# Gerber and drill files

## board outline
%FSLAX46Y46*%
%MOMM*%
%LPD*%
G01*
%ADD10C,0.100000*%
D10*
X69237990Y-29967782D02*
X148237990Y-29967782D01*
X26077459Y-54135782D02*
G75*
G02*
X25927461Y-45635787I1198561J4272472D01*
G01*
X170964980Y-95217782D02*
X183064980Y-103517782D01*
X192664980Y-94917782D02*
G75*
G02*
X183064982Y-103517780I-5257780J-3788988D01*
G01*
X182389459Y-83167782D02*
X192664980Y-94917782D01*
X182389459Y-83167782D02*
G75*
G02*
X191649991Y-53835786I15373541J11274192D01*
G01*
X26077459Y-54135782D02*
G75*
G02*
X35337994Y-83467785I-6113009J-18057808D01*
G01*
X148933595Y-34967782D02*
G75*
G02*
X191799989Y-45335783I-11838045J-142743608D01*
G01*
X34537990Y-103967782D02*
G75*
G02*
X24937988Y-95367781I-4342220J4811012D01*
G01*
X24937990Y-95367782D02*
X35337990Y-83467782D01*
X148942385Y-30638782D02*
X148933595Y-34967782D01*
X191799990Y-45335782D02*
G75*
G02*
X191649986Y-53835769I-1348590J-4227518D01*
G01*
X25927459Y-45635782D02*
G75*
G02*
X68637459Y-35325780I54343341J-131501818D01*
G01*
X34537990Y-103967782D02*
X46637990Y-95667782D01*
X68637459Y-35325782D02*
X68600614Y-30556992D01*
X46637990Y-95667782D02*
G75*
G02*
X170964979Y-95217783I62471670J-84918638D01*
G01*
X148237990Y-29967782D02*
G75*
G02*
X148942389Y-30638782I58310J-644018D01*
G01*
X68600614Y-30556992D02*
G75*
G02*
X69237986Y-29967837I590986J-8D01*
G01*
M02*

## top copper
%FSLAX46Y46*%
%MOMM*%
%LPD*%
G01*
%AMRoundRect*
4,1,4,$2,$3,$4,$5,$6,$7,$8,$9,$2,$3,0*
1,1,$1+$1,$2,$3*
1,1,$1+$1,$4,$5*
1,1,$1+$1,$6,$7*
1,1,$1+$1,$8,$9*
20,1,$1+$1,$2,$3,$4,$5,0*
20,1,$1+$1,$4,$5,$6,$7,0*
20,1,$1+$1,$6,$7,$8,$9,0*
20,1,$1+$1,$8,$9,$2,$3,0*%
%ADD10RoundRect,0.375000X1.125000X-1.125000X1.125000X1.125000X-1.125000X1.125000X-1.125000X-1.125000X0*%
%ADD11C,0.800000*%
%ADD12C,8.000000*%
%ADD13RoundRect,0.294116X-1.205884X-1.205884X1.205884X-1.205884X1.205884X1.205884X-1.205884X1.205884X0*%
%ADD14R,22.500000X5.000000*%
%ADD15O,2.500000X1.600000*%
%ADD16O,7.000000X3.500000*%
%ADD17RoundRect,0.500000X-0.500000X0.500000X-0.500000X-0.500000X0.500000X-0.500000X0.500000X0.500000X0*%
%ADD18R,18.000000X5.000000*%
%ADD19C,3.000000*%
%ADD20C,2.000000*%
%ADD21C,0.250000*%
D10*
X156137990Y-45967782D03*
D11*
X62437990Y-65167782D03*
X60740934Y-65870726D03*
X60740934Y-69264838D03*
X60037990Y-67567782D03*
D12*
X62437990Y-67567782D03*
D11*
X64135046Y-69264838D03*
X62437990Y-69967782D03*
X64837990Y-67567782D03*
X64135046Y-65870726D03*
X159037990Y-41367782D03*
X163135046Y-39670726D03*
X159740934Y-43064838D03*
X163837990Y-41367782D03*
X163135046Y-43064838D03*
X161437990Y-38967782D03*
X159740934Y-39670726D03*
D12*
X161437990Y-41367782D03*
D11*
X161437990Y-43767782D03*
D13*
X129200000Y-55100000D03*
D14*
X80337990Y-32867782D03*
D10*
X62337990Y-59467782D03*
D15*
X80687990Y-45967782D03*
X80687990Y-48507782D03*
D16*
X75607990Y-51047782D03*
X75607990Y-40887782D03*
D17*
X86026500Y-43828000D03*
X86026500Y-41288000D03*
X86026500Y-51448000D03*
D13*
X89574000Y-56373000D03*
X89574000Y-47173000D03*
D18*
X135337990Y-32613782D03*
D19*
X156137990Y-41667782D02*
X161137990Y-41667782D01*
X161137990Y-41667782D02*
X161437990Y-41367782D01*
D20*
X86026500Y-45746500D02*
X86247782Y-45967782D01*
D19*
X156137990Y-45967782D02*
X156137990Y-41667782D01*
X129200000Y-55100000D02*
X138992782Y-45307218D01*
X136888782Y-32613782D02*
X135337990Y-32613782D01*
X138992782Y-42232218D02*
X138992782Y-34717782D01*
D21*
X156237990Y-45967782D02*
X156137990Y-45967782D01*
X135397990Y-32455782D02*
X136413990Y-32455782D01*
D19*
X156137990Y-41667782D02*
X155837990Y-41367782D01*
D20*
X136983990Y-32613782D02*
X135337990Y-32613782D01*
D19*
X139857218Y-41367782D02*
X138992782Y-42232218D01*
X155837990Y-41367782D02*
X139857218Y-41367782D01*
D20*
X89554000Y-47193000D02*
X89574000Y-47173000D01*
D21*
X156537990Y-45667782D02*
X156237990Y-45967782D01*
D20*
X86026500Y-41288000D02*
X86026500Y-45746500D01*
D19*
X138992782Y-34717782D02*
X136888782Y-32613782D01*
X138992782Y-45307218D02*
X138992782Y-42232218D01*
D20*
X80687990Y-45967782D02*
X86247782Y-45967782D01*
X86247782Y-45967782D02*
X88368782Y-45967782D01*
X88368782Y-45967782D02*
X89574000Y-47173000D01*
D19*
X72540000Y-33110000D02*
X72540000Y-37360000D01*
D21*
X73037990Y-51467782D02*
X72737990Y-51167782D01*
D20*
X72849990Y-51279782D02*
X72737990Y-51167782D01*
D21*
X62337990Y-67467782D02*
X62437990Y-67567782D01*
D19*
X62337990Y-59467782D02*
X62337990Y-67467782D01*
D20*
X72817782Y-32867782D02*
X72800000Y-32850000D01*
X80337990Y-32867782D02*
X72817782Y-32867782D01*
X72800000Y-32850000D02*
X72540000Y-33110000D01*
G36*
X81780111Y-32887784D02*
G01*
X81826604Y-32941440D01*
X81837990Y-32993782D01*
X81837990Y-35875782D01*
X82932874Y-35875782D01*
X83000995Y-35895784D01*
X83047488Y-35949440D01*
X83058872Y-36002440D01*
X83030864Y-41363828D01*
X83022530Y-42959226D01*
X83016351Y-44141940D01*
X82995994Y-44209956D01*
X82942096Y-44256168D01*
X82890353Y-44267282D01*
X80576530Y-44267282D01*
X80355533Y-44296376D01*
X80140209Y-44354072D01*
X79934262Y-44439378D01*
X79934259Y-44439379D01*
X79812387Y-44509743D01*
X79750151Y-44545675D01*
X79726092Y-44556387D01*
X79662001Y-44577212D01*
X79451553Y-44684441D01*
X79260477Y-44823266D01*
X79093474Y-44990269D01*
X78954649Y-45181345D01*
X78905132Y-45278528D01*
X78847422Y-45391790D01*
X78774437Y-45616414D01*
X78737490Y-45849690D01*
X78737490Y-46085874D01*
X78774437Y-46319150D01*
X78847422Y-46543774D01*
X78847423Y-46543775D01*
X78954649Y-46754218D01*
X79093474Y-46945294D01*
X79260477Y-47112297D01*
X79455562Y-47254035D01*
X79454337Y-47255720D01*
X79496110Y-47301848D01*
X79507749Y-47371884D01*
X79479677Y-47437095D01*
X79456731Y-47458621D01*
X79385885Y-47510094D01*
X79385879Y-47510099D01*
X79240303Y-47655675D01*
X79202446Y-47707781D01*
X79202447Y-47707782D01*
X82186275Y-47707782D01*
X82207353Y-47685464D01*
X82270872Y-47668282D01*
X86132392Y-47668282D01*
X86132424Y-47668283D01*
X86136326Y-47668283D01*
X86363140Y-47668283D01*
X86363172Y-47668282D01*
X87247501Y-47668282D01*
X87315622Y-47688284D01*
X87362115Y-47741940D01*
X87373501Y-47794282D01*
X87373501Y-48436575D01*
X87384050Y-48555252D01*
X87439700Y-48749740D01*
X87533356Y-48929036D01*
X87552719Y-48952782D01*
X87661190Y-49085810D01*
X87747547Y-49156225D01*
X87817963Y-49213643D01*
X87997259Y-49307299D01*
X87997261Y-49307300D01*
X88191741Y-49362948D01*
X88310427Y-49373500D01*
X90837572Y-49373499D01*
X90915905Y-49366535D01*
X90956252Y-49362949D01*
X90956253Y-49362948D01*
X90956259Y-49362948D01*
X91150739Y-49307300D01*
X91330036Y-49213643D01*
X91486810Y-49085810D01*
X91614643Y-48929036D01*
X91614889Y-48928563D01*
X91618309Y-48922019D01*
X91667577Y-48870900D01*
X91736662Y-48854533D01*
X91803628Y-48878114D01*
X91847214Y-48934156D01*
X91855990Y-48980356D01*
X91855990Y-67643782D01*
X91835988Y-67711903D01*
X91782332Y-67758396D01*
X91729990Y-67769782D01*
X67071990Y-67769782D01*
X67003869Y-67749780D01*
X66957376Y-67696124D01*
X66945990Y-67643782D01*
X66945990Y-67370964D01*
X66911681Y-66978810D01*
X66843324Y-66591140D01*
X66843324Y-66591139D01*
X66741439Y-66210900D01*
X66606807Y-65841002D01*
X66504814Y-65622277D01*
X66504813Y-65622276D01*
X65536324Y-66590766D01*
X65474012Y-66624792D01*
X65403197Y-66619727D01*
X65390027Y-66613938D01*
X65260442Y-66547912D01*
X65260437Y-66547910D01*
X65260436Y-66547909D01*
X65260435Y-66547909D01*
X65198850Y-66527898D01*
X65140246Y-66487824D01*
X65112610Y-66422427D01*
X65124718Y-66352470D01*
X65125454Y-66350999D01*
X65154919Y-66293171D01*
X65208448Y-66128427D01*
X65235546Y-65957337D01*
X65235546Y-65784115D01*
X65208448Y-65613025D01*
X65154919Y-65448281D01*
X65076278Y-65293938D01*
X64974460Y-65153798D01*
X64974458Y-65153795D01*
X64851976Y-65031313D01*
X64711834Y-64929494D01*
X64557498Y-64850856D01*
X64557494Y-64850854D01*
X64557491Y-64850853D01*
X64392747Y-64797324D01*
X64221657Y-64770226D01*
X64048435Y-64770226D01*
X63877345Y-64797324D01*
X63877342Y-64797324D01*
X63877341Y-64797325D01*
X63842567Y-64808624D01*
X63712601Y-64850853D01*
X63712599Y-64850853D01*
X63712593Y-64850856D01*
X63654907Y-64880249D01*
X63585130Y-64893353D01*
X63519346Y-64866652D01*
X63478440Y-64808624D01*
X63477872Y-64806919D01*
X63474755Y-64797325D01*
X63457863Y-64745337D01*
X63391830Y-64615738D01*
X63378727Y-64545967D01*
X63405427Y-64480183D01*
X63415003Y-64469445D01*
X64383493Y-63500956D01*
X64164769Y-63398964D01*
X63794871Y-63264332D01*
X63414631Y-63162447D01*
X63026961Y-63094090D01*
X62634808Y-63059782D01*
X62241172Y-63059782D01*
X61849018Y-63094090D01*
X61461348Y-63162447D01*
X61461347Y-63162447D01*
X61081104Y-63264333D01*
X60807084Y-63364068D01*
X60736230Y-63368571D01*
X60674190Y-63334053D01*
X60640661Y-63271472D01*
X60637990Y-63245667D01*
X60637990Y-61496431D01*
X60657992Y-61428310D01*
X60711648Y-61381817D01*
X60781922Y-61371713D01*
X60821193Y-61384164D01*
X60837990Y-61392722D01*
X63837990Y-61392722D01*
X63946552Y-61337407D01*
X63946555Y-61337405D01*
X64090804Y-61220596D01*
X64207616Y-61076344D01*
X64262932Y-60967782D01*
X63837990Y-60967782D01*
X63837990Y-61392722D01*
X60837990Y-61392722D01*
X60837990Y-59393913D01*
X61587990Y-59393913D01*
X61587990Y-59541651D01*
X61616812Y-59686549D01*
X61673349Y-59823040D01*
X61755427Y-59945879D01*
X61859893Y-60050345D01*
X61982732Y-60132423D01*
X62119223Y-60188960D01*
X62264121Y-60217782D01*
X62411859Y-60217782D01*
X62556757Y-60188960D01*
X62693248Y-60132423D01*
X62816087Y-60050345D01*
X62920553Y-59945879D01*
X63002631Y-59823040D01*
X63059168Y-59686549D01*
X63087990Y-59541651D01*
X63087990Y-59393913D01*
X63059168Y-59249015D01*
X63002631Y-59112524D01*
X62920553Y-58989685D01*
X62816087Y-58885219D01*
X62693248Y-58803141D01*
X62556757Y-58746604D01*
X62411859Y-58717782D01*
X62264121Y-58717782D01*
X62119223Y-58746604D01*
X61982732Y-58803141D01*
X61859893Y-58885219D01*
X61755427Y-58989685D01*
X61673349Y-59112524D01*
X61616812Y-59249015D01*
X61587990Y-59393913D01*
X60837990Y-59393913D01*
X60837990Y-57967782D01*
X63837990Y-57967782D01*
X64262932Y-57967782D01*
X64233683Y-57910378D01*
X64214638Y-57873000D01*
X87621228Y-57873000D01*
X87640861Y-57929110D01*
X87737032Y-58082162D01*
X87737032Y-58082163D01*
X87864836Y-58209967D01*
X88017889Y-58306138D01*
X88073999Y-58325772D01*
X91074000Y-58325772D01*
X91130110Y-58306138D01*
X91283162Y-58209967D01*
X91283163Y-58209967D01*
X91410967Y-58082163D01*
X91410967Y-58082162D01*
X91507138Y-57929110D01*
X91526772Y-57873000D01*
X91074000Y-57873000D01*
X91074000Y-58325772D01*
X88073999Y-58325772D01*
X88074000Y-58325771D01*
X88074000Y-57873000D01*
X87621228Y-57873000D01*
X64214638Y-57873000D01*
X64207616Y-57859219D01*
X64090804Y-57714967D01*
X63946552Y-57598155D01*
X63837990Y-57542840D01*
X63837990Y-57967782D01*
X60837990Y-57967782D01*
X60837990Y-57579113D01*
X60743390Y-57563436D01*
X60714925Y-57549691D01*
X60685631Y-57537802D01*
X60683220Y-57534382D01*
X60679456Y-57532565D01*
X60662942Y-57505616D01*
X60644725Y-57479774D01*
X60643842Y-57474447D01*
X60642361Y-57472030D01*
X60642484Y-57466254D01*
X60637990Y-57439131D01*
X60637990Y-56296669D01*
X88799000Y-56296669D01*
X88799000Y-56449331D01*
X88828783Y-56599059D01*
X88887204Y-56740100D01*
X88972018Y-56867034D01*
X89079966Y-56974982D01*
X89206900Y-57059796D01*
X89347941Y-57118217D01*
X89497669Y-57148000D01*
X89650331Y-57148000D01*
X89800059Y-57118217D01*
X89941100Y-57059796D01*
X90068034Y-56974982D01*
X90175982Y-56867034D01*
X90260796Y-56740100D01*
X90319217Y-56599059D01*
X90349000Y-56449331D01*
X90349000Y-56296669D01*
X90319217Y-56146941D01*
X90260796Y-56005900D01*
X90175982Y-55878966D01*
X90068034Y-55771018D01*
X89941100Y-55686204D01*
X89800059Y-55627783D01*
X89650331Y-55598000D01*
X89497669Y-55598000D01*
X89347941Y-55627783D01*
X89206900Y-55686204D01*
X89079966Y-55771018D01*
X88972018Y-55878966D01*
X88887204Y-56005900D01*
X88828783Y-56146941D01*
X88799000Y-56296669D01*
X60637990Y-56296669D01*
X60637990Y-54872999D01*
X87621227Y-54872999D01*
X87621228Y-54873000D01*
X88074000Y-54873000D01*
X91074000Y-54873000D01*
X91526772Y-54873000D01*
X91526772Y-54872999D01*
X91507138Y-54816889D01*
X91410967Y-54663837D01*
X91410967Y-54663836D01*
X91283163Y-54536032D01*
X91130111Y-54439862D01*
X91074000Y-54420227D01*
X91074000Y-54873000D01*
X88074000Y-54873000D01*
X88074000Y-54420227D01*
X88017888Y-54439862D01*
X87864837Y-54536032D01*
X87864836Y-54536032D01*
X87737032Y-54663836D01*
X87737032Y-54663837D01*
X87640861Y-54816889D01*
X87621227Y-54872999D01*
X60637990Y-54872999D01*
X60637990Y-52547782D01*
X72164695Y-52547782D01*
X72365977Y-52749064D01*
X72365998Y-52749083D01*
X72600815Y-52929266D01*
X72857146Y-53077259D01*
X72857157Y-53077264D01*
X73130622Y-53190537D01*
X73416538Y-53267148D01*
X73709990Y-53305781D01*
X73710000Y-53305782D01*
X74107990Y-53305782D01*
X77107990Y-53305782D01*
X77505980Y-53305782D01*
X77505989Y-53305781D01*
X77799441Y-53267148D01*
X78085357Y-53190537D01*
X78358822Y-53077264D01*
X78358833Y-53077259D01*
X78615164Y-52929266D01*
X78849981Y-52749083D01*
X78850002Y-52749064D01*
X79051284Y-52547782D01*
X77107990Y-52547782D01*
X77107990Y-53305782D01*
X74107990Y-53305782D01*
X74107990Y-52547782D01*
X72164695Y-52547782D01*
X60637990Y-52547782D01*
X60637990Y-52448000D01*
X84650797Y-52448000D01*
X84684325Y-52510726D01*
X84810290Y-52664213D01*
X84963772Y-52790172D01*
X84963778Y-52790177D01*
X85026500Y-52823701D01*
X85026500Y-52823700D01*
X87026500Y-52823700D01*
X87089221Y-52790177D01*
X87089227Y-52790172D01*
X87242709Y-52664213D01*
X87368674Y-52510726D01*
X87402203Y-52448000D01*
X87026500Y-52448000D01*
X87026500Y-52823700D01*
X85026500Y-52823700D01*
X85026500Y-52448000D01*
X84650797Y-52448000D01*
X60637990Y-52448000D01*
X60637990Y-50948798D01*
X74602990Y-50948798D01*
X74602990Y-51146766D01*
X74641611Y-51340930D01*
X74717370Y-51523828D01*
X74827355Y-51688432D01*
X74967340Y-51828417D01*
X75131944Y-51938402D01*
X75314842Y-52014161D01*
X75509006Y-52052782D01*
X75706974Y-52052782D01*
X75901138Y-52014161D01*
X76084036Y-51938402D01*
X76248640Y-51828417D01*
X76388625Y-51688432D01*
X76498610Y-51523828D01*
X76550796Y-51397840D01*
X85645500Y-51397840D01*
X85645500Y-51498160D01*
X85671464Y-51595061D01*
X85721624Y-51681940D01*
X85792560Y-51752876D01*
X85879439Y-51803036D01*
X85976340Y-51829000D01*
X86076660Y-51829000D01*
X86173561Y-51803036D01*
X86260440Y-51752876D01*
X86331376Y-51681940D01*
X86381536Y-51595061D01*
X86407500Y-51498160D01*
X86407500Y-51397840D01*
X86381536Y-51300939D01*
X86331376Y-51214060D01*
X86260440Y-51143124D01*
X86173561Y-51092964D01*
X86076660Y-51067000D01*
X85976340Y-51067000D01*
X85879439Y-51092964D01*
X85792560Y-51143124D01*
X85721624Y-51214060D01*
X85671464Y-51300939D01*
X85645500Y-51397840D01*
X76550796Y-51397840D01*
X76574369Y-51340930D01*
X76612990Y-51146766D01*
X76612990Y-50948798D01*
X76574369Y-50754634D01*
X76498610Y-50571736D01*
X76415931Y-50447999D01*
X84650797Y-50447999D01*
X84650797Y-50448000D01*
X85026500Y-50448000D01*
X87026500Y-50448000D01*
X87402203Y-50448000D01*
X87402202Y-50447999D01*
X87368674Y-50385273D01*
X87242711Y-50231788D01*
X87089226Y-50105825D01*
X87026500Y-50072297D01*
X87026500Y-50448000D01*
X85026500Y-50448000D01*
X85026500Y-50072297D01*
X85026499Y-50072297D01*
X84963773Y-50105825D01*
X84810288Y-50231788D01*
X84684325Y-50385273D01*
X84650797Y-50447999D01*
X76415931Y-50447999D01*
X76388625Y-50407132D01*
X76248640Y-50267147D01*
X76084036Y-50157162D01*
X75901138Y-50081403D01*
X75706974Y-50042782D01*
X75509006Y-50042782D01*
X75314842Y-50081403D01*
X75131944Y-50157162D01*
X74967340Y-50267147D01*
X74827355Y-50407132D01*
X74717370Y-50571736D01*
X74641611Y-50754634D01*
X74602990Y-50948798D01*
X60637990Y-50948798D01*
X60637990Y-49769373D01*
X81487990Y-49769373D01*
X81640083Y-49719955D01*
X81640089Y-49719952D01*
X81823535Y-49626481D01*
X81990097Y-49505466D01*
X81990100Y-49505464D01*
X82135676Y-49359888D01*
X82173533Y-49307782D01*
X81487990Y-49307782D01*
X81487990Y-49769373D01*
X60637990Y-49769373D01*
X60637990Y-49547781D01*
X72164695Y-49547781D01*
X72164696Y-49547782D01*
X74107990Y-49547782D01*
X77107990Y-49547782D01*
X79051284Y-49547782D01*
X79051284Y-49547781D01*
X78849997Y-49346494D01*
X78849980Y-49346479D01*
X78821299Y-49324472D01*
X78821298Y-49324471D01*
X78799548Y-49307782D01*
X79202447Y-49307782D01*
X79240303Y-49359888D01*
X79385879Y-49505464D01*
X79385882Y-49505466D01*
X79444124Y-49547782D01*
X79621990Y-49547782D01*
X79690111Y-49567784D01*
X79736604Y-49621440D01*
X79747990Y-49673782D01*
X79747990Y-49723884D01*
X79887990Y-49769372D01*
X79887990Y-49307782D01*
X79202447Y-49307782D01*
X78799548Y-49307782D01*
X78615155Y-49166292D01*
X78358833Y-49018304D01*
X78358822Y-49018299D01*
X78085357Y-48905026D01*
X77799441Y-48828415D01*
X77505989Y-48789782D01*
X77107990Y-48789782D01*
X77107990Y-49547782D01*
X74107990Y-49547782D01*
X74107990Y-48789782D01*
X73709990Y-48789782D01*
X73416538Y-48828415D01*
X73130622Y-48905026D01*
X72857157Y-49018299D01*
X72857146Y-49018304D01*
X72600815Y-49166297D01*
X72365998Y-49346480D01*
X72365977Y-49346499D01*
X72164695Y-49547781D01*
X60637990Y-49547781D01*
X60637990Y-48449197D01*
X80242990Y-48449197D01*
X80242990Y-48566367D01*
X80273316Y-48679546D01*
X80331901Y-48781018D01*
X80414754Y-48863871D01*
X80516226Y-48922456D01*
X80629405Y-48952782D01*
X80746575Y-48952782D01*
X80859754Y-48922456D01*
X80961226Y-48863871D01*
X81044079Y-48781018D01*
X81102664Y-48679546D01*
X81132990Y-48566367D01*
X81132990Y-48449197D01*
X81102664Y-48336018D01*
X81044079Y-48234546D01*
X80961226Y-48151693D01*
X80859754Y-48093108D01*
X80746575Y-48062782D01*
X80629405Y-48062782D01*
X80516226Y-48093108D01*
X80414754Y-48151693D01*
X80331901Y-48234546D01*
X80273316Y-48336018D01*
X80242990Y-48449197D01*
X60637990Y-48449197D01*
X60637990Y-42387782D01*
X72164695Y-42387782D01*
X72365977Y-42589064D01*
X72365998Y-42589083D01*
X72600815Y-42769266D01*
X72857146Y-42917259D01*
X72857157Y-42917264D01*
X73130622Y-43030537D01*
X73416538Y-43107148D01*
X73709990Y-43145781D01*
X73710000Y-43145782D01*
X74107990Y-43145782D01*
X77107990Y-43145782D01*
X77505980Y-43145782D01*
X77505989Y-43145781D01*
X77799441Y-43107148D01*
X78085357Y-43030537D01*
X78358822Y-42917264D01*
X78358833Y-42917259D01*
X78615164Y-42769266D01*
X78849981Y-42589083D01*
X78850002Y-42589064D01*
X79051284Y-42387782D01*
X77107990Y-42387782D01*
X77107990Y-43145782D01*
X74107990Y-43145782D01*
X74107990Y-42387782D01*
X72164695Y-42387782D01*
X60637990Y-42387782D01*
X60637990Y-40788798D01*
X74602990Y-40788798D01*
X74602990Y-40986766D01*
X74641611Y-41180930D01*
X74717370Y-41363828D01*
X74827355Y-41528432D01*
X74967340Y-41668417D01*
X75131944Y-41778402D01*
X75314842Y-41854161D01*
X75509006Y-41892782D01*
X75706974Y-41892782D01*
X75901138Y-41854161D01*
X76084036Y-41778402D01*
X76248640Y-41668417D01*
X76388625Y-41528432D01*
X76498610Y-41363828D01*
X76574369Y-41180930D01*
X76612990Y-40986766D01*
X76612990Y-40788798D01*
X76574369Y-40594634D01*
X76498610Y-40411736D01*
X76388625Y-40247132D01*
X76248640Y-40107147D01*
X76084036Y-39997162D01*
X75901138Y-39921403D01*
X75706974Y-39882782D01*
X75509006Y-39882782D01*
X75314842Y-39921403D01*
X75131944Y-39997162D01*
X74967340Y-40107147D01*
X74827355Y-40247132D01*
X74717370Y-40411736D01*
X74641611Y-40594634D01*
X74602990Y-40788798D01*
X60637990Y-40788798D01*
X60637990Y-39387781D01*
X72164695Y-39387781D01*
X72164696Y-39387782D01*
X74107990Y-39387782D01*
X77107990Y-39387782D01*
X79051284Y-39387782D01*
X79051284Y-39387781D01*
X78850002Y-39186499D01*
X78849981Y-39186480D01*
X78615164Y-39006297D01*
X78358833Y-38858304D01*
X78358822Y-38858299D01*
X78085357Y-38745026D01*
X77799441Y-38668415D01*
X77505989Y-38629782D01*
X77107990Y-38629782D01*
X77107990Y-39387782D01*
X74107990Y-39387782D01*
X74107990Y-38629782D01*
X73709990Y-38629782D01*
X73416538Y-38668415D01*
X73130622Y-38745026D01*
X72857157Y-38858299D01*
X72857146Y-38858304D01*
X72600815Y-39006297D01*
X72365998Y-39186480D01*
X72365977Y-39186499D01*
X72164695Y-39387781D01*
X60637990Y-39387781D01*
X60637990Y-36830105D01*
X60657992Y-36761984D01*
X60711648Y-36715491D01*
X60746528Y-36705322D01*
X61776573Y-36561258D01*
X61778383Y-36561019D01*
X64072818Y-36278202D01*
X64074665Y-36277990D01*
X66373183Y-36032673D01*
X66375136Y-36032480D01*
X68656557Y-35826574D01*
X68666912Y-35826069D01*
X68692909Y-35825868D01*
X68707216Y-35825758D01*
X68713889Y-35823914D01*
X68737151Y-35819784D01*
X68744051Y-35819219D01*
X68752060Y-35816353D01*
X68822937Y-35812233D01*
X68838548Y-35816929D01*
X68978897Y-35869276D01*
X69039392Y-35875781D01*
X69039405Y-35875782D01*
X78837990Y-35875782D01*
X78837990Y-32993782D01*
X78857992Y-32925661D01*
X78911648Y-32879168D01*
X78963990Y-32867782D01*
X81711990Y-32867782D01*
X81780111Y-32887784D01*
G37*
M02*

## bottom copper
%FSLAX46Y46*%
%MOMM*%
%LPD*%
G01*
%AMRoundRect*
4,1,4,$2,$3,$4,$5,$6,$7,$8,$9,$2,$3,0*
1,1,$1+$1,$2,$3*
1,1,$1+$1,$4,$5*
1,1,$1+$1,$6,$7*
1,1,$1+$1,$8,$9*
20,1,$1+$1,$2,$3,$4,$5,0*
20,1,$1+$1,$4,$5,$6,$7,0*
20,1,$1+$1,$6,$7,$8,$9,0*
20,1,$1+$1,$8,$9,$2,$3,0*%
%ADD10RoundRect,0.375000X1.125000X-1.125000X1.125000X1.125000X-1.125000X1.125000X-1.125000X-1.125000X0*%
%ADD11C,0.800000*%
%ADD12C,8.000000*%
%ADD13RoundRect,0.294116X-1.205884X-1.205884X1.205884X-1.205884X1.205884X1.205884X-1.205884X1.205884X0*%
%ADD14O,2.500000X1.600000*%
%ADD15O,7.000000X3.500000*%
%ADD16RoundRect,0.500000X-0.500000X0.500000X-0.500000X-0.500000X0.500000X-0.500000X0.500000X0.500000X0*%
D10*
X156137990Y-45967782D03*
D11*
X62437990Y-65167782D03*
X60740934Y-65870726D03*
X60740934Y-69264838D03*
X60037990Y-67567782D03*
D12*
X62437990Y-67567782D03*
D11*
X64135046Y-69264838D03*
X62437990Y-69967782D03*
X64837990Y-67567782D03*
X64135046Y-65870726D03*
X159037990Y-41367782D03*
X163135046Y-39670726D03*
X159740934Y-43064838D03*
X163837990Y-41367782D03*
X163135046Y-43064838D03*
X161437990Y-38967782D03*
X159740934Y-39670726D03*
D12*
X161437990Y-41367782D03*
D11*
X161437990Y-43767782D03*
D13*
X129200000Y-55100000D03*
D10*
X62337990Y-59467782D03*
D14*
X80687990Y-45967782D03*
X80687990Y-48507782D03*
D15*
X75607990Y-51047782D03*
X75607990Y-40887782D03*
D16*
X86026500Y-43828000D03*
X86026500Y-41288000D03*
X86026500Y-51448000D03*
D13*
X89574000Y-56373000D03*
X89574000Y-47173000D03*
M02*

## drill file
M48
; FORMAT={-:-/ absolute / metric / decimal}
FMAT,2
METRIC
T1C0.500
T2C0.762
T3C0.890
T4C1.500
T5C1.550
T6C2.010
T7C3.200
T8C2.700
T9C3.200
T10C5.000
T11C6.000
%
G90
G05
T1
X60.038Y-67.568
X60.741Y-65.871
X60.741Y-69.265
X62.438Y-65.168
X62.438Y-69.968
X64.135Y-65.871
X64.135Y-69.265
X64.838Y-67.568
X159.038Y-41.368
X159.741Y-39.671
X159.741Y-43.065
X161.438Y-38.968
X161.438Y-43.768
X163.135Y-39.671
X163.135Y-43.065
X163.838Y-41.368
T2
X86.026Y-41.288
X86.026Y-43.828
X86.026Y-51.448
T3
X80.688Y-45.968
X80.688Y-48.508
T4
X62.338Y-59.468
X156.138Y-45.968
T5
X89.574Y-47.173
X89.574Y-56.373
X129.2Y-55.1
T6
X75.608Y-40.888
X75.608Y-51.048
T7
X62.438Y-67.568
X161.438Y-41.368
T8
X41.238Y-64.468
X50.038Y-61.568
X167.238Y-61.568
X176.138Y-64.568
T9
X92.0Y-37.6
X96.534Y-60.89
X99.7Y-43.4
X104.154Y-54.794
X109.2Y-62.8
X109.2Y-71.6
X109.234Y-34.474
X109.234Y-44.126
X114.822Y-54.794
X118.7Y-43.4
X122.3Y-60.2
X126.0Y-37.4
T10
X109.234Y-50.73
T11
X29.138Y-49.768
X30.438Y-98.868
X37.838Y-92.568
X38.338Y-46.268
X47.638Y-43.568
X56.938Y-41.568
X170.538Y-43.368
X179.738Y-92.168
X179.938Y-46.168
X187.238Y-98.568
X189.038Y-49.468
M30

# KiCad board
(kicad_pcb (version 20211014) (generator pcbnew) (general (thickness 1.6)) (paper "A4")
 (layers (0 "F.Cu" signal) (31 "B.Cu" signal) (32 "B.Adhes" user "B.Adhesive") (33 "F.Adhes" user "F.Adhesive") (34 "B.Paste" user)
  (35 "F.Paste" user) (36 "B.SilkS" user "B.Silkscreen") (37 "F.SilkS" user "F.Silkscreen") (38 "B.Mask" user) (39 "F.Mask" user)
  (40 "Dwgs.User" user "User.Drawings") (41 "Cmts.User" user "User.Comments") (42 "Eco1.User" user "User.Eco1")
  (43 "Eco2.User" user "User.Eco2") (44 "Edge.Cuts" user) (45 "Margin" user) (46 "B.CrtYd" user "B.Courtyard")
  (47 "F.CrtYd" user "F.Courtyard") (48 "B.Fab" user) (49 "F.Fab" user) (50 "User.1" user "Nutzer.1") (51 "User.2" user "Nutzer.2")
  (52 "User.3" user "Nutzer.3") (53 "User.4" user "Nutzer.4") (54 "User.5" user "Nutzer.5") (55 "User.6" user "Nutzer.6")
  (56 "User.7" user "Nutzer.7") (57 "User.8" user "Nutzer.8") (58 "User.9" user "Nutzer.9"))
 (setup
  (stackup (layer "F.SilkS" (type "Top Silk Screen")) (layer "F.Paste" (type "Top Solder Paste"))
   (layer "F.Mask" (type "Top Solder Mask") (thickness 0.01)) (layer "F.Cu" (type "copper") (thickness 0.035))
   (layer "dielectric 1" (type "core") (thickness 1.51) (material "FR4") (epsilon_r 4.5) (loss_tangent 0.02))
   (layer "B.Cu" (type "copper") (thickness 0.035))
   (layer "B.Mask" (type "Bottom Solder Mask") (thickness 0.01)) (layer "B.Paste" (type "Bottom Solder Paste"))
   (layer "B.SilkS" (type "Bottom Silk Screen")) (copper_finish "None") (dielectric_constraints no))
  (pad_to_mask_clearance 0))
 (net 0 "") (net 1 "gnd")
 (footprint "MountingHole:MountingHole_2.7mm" (layer "F.Cu") (at 50.03799 61.567782)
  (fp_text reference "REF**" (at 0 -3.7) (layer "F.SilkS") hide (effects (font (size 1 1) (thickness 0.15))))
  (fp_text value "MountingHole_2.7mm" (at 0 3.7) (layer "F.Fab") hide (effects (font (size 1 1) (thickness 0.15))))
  (pad "" np_thru_hole circle (at 0 0) (size 2.7 2.7) (drill 2.7) (layers *.Cu *.Mask)))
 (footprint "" (layer "F.Cu") (at 156.13799 45.967782)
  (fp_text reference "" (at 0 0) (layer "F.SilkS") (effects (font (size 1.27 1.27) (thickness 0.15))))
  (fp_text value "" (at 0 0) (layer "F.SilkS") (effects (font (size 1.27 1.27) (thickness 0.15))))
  (pad "1" thru_hole roundrect (at 0 0 90) (size 3 3) (drill 1.5) (layers *.Cu *.Mask) (roundrect_rratio 0.125)))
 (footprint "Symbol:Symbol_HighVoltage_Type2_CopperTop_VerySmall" (layer "F.Cu") (at 165.13799 49.467782)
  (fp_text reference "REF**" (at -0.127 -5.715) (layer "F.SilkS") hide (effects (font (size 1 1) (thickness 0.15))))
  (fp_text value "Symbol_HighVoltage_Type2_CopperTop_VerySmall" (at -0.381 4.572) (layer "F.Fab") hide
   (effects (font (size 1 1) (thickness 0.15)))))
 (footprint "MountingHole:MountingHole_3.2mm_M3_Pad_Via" (layer "F.Cu") (at 62.43799 67.567782)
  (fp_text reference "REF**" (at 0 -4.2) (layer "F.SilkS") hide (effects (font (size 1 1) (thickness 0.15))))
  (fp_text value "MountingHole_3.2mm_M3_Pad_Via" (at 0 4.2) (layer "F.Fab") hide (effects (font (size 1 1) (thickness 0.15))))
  (pad "1" thru_hole circle (at 0 -2.4) (size 0.8 0.8) (drill 0.5) (layers *.Cu *.Mask))
  (pad "1" thru_hole circle (at -1.697056 -1.697056) (size 0.8 0.8) (drill 0.5) (layers *.Cu *.Mask))
  (pad "1" thru_hole circle (at -1.697056 1.697056) (size 0.8 0.8) (drill 0.5) (layers *.Cu *.Mask))
  (pad "1" thru_hole circle (at -2.4 0) (size 0.8 0.8) (drill 0.5) (layers *.Cu *.Mask))
  (pad "1" thru_hole circle (at 0 0) (size 8 8) (drill 3.2) (layers *.Cu *.Mask) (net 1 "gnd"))
  (pad "1" thru_hole circle (at 1.697056 1.697056) (size 0.8 0.8) (drill 0.5) (layers *.Cu *.Mask))
  (pad "1" thru_hole circle (at 0 2.4) (size 0.8 0.8) (drill 0.5) (layers *.Cu *.Mask))
  (pad "1" thru_hole circle (at 2.4 0) (size 0.8 0.8) (drill 0.5) (layers *.Cu *.Mask))
  (pad "1" thru_hole circle (at 1.697056 -1.697056) (size 0.8 0.8) (drill 0.5) (layers *.Cu *.Mask)))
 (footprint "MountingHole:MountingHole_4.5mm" (layer "F.Cu") (at 37.83799 92.567782)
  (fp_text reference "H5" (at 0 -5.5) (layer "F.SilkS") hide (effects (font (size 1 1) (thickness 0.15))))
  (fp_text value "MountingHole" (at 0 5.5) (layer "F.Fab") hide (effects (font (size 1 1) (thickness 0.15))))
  (pad "" np_thru_hole circle (at 0 0) (size 6 6) (drill 6) (layers F&B.Cu *.Mask)))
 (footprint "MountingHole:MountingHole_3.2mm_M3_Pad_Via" (layer "F.Cu") (at 161.43799 41.367782)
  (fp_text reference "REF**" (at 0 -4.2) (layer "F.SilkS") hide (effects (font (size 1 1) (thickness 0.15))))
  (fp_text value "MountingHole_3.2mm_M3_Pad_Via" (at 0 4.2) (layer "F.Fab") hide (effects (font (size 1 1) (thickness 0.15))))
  (pad "1" thru_hole circle (at -2.4 0) (size 0.8 0.8) (drill 0.5) (layers *.Cu *.Mask))
  (pad "1" thru_hole circle (at 1.697056 -1.697056) (size 0.8 0.8) (drill 0.5) (layers *.Cu *.Mask))
  (pad "1" thru_hole circle (at -1.697056 1.697056) (size 0.8 0.8) (drill 0.5) (layers *.Cu *.Mask))
  (pad "1" thru_hole circle (at 2.4 0) (size 0.8 0.8) (drill 0.5) (layers *.Cu *.Mask))
  (pad "1" thru_hole circle (at 1.697056 1.697056) (size 0.8 0.8) (drill 0.5) (layers *.Cu *.Mask))
  (pad "1" thru_hole circle (at 0 -2.4) (size 0.8 0.8) (drill 0.5) (layers *.Cu *.Mask))
  (pad "1" thru_hole circle (at -1.697056 -1.697056) (size 0.8 0.8) (drill 0.5) (layers *.Cu *.Mask))
  (pad "1" thru_hole circle (at 0 0) (size 8 8) (drill 3.2) (layers *.Cu *.Mask))
  (pad "1" thru_hole circle (at 0 2.4) (size 0.8 0.8) (drill 0.5) (layers *.Cu *.Mask)))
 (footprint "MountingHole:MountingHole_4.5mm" (layer "F.Cu") (at 30.43799 98.867782)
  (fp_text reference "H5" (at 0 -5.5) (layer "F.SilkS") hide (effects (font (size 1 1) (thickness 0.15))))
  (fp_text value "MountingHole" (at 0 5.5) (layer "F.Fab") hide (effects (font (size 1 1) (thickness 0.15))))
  (pad "" np_thru_hole circle (at 0 0) (size 6 6) (drill 6) (layers F&B.Cu *.Mask)))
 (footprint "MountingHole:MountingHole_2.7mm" (layer "F.Cu") (at 176.13799 64.567782)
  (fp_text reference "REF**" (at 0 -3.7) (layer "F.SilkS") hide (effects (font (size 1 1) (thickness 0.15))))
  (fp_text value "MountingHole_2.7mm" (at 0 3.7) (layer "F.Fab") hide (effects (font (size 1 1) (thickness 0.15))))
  (pad "" np_thru_hole circle (at 0 0) (size 2.7 2.7) (drill 2.7) (layers *.Cu *.Mask)))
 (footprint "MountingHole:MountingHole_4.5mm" (layer "F.Cu") (at 179.73799 92.167782)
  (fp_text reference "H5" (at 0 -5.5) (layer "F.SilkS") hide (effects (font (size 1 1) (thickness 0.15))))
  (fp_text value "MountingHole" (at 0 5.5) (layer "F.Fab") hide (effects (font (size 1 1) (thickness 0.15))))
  (pad "" np_thru_hole circle (at 0 0) (size 6 6) (drill 6) (layers F&B.Cu *.Mask)))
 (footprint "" (layer "F.Cu") (at 129.2 55.1)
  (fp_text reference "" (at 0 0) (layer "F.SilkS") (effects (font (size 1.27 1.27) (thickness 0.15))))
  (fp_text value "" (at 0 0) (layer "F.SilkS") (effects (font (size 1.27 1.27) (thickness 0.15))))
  (pad "5" thru_hole roundrect (at 0 0) (size 3 3) (drill 1.55) (layers *.Cu *.Mask) (roundrect_rratio 0.09803882353)))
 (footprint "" (layer "F.Cu") (at 109.234 44.126)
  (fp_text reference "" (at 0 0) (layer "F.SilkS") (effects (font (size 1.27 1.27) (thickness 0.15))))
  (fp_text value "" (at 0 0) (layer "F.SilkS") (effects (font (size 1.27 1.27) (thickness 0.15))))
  (pad "" np_thru_hole circle (at 0 0) (size 3.2 3.2) (drill 3.2) (layers *.Cu *.Mask)))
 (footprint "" (layer "F.Cu") (at 126 37.4)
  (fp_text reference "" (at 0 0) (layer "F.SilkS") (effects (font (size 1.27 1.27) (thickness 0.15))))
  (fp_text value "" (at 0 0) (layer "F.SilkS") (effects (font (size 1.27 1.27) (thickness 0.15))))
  (pad "" np_thru_hole circle (at 0 0) (size 3.2 3.2) (drill 3.2) (layers *.Cu *.Mask)))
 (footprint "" (layer "F.Cu") (at 109.2 62.8)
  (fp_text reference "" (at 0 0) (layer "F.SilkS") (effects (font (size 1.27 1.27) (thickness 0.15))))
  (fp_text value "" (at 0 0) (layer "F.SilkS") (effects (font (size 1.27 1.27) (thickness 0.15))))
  (pad "" np_thru_hole circle (at 0 0) (size 3.2 3.2) (drill 3.2) (layers *.Cu *.Mask)))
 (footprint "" (layer "F.Cu") (at 96.534 60.89)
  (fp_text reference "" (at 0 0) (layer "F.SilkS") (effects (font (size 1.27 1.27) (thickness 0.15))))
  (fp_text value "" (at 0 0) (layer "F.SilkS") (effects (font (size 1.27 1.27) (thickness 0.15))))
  (pad "" np_thru_hole circle (at 0 0) (size 3.2 3.2) (drill 3.2) (layers *.Cu *.Mask)))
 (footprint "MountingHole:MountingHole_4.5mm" (layer "F.Cu") (at 47.63799 43.567782)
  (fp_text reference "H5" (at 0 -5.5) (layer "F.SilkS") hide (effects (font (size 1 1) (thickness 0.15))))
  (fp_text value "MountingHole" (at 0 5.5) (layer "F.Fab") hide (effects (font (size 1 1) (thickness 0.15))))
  (pad "" np_thru_hole circle (at 0 0) (size 6 6) (drill 6) (layers F&B.Cu *.Mask)))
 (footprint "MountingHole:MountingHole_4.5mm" (layer "F.Cu") (at 189.03799 49.467782)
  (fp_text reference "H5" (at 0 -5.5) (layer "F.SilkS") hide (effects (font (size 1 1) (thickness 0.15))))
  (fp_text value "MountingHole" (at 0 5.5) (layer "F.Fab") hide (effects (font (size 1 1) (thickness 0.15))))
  (pad "" np_thru_hole circle (at 0 0) (size 6 6) (drill 6) (layers F&B.Cu *.Mask)))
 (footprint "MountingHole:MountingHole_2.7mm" (layer "F.Cu") (at 167.23799 61.567782)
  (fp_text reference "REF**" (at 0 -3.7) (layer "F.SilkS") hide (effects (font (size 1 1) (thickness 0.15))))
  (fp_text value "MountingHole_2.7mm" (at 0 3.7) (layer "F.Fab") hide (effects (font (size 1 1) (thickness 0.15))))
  (pad "" np_thru_hole circle (at 0 0) (size 2.7 2.7) (drill 2.7) (layers *.Cu *.Mask)))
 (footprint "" (layer "F.Cu") (at 80.33799 32.867782)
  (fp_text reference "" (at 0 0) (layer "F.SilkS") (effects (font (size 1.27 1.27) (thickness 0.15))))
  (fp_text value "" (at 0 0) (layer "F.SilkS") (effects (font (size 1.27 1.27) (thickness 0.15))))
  (pad "1" smd rect (at 0 0 180) (size 22.5 5) (layers "F.Cu" "F.Mask") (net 1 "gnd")))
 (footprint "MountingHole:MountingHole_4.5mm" (layer "F.Cu") (at 29.13799 49.767782)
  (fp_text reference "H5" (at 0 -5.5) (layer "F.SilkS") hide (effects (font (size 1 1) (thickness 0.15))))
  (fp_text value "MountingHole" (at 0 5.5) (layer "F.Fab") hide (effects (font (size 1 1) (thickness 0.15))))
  (pad "" np_thru_hole circle (at 0 0) (size 6 6) (drill 6) (layers F&B.Cu *.Mask)))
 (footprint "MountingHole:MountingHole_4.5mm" (layer "F.Cu") (at 187.23799 98.567782)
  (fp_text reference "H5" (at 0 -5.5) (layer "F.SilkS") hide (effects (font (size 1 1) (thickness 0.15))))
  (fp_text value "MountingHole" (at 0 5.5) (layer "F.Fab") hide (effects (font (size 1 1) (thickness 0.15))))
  (pad "" np_thru_hole circle (at 0 0) (size 6 6) (drill 6) (layers F&B.Cu *.Mask)))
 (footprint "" (layer "F.Cu") (at 122.3 60.2)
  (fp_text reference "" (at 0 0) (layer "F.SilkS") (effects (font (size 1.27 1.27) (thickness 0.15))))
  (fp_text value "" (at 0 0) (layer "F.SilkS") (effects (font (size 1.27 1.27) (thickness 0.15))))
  (pad "" np_thru_hole circle (at 0 0) (size 3.2 3.2) (drill 3.2) (layers *.Cu *.Mask)))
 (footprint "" (layer "F.Cu") (at 104.154 54.794)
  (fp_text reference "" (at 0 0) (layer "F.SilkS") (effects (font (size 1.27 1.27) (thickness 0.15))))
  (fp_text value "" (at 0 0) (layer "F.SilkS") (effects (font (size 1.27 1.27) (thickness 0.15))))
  (pad "" np_thru_hole circle (at 0 0) (size 3.2 3.2) (drill 3.2) (layers *.Cu *.Mask)))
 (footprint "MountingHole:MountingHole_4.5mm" (layer "F.Cu") (at 56.93799 41.567782)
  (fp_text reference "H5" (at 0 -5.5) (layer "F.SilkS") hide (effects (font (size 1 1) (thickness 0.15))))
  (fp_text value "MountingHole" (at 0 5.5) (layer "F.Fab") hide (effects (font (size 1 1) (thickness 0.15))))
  (pad "" np_thru_hole circle (at 0 0) (size 6 6) (drill 6) (layers F&B.Cu *.Mask)))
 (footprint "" (layer "F.Cu") (at 109.2 71.6)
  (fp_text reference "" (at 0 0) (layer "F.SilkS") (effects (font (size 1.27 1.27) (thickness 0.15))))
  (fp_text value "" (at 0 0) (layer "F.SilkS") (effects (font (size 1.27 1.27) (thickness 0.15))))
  (pad "" np_thru_hole circle (at 0 0) (size 3.2 3.2) (drill 3.2) (layers *.Cu *.Mask)))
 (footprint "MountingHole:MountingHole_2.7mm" (layer "F.Cu") (at 41.23799 64.467782)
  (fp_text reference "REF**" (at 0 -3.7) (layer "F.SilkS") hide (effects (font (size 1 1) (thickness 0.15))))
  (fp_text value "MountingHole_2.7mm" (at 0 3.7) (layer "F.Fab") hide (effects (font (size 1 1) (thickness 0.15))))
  (pad "" np_thru_hole circle (at 0 0) (size 2.7 2.7) (drill 2.7) (layers *.Cu *.Mask)))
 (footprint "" (layer "F.Cu") (at 109.234 34.474)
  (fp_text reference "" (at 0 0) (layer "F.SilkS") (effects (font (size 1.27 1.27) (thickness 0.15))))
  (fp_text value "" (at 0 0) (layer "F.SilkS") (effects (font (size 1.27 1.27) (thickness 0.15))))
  (pad "" np_thru_hole circle (at 0 0) (size 3.2 3.2) (drill 3.2) (layers *.Cu *.Mask)))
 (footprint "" (layer "F.Cu") (at 62.33799 59.467782)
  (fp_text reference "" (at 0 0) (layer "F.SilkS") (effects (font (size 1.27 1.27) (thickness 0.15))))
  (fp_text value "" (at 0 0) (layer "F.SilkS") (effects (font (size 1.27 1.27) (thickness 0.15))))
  (pad "1" thru_hole roundrect (at 0 0 90) (size 3 3) (drill 1.5) (layers *.Cu *.Mask) (roundrect_rratio 0.125) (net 1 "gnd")))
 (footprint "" (layer "F.Cu") (at 99.7 43.4)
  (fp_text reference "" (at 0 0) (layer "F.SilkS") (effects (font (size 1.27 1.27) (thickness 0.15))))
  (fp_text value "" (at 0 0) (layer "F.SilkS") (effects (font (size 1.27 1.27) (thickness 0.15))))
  (pad "" np_thru_hole circle (at 0 0) (size 3.2 3.2) (drill 3.2) (layers *.Cu *.Mask)))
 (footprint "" (layer "F.Cu") (at 109.234 50.73)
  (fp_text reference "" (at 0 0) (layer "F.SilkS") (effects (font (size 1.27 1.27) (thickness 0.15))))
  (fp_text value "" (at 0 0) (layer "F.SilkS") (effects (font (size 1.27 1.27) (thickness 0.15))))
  (pad "" np_thru_hole circle (at 0 0) (size 5 5) (drill 5) (layers F&B.Cu *.Mask)))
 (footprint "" (layer "F.Cu") (at 92 37.6)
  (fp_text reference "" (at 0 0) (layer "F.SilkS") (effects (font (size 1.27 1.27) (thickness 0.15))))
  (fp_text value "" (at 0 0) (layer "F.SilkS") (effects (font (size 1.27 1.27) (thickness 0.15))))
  (pad "" np_thru_hole circle (at 0 0) (size 3.2 3.2) (drill 3.2) (layers *.Cu *.Mask)))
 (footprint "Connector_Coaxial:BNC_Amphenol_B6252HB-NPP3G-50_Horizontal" (layer "F.Cu") (at 80.68799 45.967782 90)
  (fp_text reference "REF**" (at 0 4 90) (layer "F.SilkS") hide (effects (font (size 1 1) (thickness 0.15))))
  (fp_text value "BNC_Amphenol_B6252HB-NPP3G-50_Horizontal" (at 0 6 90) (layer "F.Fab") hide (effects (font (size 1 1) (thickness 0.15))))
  (pad "1" thru_hole oval (at 0 0 90) (size 1.6 2.5) (drill 0.89) (layers *.Cu *.Mask))
  (pad "2" thru_hole oval (at -2.54 0 90) (size 1.6 2.5) (drill 0.89) (layers *.Cu *.Mask) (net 1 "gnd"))
  (pad "2" thru_hole oval (at -5.08 -5.08 90) (size 3.5 7) (drill 2.01) (layers *.Cu *.Mask) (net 1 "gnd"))
  (pad "2" thru_hole oval (at 5.08 -5.08 90) (size 3.5 7) (drill 2.01) (layers *.Cu *.Mask) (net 1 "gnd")))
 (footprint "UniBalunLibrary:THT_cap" (layer "F.Cu") (at 86.0265 46.368 -90)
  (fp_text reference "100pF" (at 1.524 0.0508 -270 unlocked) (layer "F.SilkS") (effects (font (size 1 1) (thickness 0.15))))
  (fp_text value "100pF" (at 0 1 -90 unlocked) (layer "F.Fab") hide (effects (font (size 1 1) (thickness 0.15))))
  (pad "1" thru_hole roundrect (at -2.54 0 270) (size 2 2) (drill 0.762) (layers *.Cu *.Mask) (roundrect_rratio 0.25))
  (pad "1" thru_hole roundrect (at -5.08 0 270) (size 2 2) (drill 0.762) (layers *.Cu *.Mask) (roundrect_rratio 0.25))
  (pad "2" thru_hole roundrect (at 5.08 0 270) (size 2 2) (drill 0.762) (layers *.Cu *.Mask) (roundrect_rratio 0.25) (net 1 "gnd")))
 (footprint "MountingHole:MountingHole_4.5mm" (layer "F.Cu") (at 170.53799 43.367782)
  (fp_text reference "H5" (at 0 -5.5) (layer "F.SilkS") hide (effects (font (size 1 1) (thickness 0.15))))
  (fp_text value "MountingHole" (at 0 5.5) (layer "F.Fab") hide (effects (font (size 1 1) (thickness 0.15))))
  (pad "" np_thru_hole circle (at 0 0) (size 6 6) (drill 6) (layers F&B.Cu *.Mask)))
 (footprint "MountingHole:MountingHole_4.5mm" (layer "F.Cu") (at 38.33799 46.267782)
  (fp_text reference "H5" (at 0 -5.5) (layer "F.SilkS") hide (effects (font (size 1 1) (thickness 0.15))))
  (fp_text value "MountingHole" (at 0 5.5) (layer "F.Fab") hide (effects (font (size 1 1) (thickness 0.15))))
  (pad "" np_thru_hole circle (at 0 0) (size 6 6) (drill 6) (layers F&B.Cu *.Mask)))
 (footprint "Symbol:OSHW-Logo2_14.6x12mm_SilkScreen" (layer "F.Cu") (at 49.93799 75.467782)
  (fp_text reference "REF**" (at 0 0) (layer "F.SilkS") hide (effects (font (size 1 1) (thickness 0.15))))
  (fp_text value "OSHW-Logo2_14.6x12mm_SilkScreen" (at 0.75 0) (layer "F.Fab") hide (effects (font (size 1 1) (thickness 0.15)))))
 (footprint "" (layer "F.Cu") (at 89.574 56.373)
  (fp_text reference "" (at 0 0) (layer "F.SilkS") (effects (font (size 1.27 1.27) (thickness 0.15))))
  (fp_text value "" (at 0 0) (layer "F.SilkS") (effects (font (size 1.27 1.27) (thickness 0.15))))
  (pad "5" thru_hole roundrect (at 0 0) (size 3 3) (drill 1.55) (layers *.Cu *.Mask) (roundrect_rratio 0.09803882353) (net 1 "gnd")))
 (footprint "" (layer "F.Cu") (at 89.574 47.173)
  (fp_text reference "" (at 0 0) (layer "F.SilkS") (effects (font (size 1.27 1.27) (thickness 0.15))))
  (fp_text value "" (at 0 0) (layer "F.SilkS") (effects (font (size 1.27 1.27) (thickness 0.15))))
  (pad "1" thru_hole roundrect (at 0 0) (size 3 3) (drill 1.55) (layers *.Cu *.Mask) (roundrect_rratio 0.09803882353)))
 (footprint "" (layer "F.Cu") (at 118.7 43.4)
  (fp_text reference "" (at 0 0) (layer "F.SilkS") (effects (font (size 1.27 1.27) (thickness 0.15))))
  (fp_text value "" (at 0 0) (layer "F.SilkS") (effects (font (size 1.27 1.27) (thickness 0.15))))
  (pad "" np_thru_hole circle (at 0 0) (size 3.2 3.2) (drill 3.2) (layers *.Cu *.Mask)))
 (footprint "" (layer "F.Cu") (at 114.822 54.794)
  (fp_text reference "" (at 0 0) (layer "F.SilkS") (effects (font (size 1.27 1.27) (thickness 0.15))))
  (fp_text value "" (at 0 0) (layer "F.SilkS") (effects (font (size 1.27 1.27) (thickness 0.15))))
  (pad "" np_thru_hole circle (at 0 0) (size 3.2 3.2) (drill 3.2) (layers *.Cu *.Mask)))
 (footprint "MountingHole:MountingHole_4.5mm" (layer "F.Cu") (at 179.93799 46.167782)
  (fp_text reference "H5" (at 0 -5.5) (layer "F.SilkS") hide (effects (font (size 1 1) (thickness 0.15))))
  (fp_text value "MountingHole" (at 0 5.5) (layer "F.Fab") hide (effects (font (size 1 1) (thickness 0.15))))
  (pad "" np_thru_hole circle (at 0 0) (size 6 6) (drill 6) (layers F&B.Cu *.Mask)))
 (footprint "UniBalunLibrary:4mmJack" (layer "B.Cu") (at 135.59199 32.867782)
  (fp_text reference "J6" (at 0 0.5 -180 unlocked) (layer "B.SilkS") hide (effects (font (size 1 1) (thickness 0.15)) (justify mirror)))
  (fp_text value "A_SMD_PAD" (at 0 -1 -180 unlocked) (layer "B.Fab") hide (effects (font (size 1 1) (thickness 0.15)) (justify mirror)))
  (pad "1" smd rect (at -0.254 -0.254) (size 18 5) (layers "F.Cu" "F.Mask")))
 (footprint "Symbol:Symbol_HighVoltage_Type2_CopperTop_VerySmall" (layer "B.Cu") (at 165.33799 49.467782 180)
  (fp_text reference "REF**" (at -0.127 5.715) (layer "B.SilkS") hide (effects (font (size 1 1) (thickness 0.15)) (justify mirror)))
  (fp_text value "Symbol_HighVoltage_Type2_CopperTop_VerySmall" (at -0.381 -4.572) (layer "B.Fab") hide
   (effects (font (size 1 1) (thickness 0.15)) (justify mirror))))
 (gr_line (start 69.23799 29.967782) (end 148.23799 29.967782) (layer "Edge.Cuts") (width 0.1))
 (gr_arc (start 26.077459 54.135782) (mid 22.839303 49.941602) (end 25.927459 45.635782) (layer "Edge.Cuts") (width 0.1))
 (gr_line (start 170.96498 95.217782) (end 183.06498 103.517782) (layer "Edge.Cuts") (width 0.1))
 (gr_arc (start 192.66498 94.917782) (mid 191.731495 103.533891) (end 183.06498 103.517782) (layer "Edge.Cuts") (width 0.1))
 (gr_line (start 182.389459 83.167782) (end 192.66498 94.917782) (layer "Edge.Cuts") (width 0.1))
 (gr_arc (start 182.389459 83.167782) (mid 179.583079 66.153927) (end 191.64999 53.835782) (layer "Edge.Cuts") (width 0.1))
 (gr_arc (start 26.077459 54.135782) (mid 38.14437 66.453927) (end 35.33799 83.467782) (layer "Edge.Cuts") (width 0.1))
 (gr_arc (start 148.933595 34.967782) (mid 170.768231 38.492039) (end 191.79999 45.335782) (layer "Edge.Cuts") (width 0.1))
 (gr_arc (start 34.53799 103.967782) (mid 25.871475 103.983891) (end 24.93799 95.367782) (layer "Edge.Cuts") (width 0.1))
 (gr_line (start 24.93799 95.367782) (end 35.33799 83.467782) (layer "Edge.Cuts") (width 0.1))
 (gr_line (start 148.942385 30.638782) (end 148.933595 34.967782) (layer "Edge.Cuts") (width 0.1))
 (gr_arc (start 191.79999 45.335782) (mid 194.888146 49.641602) (end 191.64999 53.835782) (layer "Edge.Cuts") (width 0.1))
 (gr_arc (start 25.927459 45.635782) (mid 46.882109 38.822301) (end 68.637459 35.325782) (layer "Edge.Cuts") (width 0.1))
 (gr_line (start 34.53799 103.967782) (end 46.63799 95.667782) (layer "Edge.Cuts") (width 0.1))
 (gr_line (start 68.637459 35.325782) (end 68.600614 30.556992) (layer "Edge.Cuts") (width 0.1))
 (gr_arc (start 46.63799 95.667782) (mid 108.728089 75.164699) (end 170.96498 95.217782) (layer "Edge.Cuts") (width 0.1))
 (gr_arc (start 148.23799 29.967782) (mid 148.742309 30.143589) (end 148.942385 30.638782) (layer "Edge.Cuts") (width 0.1))
 (gr_arc (start 68.600614 30.556992) (mid 68.790444 30.122995) (end 69.23799 29.967782) (layer "Edge.Cuts") (width 0.1))
 (segment (start 156.13799 41.667782) (end 161.13799 41.667782) (width 3) (layer "F.Cu") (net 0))
 (segment (start 161.13799 41.667782) (end 161.43799 41.367782) (width 3) (layer "F.Cu") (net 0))
 (segment (start 86.0265 45.7465) (end 86.247782 45.967782) (width 2) (layer "F.Cu") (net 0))
 (segment (start 156.13799 45.967782) (end 156.13799 41.667782) (width 3) (layer "F.Cu") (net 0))
 (segment (start 129.2 55.1) (end 138.992782 45.307218) (width 3) (layer "F.Cu") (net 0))
 (segment (start 136.888782 32.613782) (end 135.33799 32.613782) (width 3) (layer "F.Cu") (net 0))
 (segment (start 138.992782 42.232218) (end 138.992782 34.717782) (width 3) (layer "F.Cu") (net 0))
 (segment (start 156.23799 45.967782) (end 156.13799 45.967782) (width 0.25) (layer "F.Cu") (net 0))
 (segment (start 135.39799 32.455782) (end 136.41399 32.455782) (width 0.25) (layer "F.Cu") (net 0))
 (segment (start 156.13799 41.667782) (end 155.83799 41.367782) (width 3) (layer "F.Cu") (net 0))
 (segment (start 136.98399 32.613782) (end 135.33799 32.613782) (width 2) (layer "F.Cu") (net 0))
 (segment (start 139.857218 41.367782) (end 138.992782 42.232218) (width 3) (layer "F.Cu") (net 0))
 (segment (start 155.83799 41.367782) (end 139.857218 41.367782) (width 3) (layer "F.Cu") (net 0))
 (segment (start 89.554 47.193) (end 89.574 47.173) (width 2) (layer "F.Cu") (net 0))
 (segment (start 156.53799 45.667782) (end 156.23799 45.967782) (width 0.25) (layer "F.Cu") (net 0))
 (segment (start 86.0265 41.288) (end 86.0265 45.7465) (width 2) (layer "F.Cu") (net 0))
 (segment (start 138.992782 34.717782) (end 136.888782 32.613782) (width 3) (layer "F.Cu") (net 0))
 (segment (start 138.992782 45.307218) (end 138.992782 42.232218) (width 3) (layer "F.Cu") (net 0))
 (segment (start 80.68799 45.967782) (end 86.247782 45.967782) (width 2) (layer "F.Cu") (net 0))
 (segment (start 86.247782 45.967782) (end 88.368782 45.967782) (width 2) (layer "F.Cu") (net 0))
 (segment (start 88.368782 45.967782) (end 89.574 47.173) (width 2) (layer "F.Cu") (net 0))
 (segment (start 72.54 33.11) (end 72.54 37.36) (width 3) (layer "F.Cu") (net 1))
 (segment (start 73.03799 51.467782) (end 72.73799 51.167782) (width 0.25) (layer "F.Cu") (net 1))
 (segment (start 72.84999 51.279782) (end 72.73799 51.167782) (width 2) (layer "F.Cu") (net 1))
 (segment (start 62.33799 67.467782) (end 62.43799 67.567782) (width 0.25) (layer "F.Cu") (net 1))
 (segment (start 62.33799 59.467782) (end 62.33799 67.467782) (width 3) (layer "F.Cu") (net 1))
 (segment (start 72.817782 32.867782) (end 72.8 32.85) (width 2) (layer "F.Cu") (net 1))
 (segment (start 80.33799 32.867782) (end 72.817782 32.867782) (width 2) (layer "F.Cu") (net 1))
 (segment (start 72.8 32.85) (end 72.54 33.11) (width 2) (layer "F.Cu") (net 1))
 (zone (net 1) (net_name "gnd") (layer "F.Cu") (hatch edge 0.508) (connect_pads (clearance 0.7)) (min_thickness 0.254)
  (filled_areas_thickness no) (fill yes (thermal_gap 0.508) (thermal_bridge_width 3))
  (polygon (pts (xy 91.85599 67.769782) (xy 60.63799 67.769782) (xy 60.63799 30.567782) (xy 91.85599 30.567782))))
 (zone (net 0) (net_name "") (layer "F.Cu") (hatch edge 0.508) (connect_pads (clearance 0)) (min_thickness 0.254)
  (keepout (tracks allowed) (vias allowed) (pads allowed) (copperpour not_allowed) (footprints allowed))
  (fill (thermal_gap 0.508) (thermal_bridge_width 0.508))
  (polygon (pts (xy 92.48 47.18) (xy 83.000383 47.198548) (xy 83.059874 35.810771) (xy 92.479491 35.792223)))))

